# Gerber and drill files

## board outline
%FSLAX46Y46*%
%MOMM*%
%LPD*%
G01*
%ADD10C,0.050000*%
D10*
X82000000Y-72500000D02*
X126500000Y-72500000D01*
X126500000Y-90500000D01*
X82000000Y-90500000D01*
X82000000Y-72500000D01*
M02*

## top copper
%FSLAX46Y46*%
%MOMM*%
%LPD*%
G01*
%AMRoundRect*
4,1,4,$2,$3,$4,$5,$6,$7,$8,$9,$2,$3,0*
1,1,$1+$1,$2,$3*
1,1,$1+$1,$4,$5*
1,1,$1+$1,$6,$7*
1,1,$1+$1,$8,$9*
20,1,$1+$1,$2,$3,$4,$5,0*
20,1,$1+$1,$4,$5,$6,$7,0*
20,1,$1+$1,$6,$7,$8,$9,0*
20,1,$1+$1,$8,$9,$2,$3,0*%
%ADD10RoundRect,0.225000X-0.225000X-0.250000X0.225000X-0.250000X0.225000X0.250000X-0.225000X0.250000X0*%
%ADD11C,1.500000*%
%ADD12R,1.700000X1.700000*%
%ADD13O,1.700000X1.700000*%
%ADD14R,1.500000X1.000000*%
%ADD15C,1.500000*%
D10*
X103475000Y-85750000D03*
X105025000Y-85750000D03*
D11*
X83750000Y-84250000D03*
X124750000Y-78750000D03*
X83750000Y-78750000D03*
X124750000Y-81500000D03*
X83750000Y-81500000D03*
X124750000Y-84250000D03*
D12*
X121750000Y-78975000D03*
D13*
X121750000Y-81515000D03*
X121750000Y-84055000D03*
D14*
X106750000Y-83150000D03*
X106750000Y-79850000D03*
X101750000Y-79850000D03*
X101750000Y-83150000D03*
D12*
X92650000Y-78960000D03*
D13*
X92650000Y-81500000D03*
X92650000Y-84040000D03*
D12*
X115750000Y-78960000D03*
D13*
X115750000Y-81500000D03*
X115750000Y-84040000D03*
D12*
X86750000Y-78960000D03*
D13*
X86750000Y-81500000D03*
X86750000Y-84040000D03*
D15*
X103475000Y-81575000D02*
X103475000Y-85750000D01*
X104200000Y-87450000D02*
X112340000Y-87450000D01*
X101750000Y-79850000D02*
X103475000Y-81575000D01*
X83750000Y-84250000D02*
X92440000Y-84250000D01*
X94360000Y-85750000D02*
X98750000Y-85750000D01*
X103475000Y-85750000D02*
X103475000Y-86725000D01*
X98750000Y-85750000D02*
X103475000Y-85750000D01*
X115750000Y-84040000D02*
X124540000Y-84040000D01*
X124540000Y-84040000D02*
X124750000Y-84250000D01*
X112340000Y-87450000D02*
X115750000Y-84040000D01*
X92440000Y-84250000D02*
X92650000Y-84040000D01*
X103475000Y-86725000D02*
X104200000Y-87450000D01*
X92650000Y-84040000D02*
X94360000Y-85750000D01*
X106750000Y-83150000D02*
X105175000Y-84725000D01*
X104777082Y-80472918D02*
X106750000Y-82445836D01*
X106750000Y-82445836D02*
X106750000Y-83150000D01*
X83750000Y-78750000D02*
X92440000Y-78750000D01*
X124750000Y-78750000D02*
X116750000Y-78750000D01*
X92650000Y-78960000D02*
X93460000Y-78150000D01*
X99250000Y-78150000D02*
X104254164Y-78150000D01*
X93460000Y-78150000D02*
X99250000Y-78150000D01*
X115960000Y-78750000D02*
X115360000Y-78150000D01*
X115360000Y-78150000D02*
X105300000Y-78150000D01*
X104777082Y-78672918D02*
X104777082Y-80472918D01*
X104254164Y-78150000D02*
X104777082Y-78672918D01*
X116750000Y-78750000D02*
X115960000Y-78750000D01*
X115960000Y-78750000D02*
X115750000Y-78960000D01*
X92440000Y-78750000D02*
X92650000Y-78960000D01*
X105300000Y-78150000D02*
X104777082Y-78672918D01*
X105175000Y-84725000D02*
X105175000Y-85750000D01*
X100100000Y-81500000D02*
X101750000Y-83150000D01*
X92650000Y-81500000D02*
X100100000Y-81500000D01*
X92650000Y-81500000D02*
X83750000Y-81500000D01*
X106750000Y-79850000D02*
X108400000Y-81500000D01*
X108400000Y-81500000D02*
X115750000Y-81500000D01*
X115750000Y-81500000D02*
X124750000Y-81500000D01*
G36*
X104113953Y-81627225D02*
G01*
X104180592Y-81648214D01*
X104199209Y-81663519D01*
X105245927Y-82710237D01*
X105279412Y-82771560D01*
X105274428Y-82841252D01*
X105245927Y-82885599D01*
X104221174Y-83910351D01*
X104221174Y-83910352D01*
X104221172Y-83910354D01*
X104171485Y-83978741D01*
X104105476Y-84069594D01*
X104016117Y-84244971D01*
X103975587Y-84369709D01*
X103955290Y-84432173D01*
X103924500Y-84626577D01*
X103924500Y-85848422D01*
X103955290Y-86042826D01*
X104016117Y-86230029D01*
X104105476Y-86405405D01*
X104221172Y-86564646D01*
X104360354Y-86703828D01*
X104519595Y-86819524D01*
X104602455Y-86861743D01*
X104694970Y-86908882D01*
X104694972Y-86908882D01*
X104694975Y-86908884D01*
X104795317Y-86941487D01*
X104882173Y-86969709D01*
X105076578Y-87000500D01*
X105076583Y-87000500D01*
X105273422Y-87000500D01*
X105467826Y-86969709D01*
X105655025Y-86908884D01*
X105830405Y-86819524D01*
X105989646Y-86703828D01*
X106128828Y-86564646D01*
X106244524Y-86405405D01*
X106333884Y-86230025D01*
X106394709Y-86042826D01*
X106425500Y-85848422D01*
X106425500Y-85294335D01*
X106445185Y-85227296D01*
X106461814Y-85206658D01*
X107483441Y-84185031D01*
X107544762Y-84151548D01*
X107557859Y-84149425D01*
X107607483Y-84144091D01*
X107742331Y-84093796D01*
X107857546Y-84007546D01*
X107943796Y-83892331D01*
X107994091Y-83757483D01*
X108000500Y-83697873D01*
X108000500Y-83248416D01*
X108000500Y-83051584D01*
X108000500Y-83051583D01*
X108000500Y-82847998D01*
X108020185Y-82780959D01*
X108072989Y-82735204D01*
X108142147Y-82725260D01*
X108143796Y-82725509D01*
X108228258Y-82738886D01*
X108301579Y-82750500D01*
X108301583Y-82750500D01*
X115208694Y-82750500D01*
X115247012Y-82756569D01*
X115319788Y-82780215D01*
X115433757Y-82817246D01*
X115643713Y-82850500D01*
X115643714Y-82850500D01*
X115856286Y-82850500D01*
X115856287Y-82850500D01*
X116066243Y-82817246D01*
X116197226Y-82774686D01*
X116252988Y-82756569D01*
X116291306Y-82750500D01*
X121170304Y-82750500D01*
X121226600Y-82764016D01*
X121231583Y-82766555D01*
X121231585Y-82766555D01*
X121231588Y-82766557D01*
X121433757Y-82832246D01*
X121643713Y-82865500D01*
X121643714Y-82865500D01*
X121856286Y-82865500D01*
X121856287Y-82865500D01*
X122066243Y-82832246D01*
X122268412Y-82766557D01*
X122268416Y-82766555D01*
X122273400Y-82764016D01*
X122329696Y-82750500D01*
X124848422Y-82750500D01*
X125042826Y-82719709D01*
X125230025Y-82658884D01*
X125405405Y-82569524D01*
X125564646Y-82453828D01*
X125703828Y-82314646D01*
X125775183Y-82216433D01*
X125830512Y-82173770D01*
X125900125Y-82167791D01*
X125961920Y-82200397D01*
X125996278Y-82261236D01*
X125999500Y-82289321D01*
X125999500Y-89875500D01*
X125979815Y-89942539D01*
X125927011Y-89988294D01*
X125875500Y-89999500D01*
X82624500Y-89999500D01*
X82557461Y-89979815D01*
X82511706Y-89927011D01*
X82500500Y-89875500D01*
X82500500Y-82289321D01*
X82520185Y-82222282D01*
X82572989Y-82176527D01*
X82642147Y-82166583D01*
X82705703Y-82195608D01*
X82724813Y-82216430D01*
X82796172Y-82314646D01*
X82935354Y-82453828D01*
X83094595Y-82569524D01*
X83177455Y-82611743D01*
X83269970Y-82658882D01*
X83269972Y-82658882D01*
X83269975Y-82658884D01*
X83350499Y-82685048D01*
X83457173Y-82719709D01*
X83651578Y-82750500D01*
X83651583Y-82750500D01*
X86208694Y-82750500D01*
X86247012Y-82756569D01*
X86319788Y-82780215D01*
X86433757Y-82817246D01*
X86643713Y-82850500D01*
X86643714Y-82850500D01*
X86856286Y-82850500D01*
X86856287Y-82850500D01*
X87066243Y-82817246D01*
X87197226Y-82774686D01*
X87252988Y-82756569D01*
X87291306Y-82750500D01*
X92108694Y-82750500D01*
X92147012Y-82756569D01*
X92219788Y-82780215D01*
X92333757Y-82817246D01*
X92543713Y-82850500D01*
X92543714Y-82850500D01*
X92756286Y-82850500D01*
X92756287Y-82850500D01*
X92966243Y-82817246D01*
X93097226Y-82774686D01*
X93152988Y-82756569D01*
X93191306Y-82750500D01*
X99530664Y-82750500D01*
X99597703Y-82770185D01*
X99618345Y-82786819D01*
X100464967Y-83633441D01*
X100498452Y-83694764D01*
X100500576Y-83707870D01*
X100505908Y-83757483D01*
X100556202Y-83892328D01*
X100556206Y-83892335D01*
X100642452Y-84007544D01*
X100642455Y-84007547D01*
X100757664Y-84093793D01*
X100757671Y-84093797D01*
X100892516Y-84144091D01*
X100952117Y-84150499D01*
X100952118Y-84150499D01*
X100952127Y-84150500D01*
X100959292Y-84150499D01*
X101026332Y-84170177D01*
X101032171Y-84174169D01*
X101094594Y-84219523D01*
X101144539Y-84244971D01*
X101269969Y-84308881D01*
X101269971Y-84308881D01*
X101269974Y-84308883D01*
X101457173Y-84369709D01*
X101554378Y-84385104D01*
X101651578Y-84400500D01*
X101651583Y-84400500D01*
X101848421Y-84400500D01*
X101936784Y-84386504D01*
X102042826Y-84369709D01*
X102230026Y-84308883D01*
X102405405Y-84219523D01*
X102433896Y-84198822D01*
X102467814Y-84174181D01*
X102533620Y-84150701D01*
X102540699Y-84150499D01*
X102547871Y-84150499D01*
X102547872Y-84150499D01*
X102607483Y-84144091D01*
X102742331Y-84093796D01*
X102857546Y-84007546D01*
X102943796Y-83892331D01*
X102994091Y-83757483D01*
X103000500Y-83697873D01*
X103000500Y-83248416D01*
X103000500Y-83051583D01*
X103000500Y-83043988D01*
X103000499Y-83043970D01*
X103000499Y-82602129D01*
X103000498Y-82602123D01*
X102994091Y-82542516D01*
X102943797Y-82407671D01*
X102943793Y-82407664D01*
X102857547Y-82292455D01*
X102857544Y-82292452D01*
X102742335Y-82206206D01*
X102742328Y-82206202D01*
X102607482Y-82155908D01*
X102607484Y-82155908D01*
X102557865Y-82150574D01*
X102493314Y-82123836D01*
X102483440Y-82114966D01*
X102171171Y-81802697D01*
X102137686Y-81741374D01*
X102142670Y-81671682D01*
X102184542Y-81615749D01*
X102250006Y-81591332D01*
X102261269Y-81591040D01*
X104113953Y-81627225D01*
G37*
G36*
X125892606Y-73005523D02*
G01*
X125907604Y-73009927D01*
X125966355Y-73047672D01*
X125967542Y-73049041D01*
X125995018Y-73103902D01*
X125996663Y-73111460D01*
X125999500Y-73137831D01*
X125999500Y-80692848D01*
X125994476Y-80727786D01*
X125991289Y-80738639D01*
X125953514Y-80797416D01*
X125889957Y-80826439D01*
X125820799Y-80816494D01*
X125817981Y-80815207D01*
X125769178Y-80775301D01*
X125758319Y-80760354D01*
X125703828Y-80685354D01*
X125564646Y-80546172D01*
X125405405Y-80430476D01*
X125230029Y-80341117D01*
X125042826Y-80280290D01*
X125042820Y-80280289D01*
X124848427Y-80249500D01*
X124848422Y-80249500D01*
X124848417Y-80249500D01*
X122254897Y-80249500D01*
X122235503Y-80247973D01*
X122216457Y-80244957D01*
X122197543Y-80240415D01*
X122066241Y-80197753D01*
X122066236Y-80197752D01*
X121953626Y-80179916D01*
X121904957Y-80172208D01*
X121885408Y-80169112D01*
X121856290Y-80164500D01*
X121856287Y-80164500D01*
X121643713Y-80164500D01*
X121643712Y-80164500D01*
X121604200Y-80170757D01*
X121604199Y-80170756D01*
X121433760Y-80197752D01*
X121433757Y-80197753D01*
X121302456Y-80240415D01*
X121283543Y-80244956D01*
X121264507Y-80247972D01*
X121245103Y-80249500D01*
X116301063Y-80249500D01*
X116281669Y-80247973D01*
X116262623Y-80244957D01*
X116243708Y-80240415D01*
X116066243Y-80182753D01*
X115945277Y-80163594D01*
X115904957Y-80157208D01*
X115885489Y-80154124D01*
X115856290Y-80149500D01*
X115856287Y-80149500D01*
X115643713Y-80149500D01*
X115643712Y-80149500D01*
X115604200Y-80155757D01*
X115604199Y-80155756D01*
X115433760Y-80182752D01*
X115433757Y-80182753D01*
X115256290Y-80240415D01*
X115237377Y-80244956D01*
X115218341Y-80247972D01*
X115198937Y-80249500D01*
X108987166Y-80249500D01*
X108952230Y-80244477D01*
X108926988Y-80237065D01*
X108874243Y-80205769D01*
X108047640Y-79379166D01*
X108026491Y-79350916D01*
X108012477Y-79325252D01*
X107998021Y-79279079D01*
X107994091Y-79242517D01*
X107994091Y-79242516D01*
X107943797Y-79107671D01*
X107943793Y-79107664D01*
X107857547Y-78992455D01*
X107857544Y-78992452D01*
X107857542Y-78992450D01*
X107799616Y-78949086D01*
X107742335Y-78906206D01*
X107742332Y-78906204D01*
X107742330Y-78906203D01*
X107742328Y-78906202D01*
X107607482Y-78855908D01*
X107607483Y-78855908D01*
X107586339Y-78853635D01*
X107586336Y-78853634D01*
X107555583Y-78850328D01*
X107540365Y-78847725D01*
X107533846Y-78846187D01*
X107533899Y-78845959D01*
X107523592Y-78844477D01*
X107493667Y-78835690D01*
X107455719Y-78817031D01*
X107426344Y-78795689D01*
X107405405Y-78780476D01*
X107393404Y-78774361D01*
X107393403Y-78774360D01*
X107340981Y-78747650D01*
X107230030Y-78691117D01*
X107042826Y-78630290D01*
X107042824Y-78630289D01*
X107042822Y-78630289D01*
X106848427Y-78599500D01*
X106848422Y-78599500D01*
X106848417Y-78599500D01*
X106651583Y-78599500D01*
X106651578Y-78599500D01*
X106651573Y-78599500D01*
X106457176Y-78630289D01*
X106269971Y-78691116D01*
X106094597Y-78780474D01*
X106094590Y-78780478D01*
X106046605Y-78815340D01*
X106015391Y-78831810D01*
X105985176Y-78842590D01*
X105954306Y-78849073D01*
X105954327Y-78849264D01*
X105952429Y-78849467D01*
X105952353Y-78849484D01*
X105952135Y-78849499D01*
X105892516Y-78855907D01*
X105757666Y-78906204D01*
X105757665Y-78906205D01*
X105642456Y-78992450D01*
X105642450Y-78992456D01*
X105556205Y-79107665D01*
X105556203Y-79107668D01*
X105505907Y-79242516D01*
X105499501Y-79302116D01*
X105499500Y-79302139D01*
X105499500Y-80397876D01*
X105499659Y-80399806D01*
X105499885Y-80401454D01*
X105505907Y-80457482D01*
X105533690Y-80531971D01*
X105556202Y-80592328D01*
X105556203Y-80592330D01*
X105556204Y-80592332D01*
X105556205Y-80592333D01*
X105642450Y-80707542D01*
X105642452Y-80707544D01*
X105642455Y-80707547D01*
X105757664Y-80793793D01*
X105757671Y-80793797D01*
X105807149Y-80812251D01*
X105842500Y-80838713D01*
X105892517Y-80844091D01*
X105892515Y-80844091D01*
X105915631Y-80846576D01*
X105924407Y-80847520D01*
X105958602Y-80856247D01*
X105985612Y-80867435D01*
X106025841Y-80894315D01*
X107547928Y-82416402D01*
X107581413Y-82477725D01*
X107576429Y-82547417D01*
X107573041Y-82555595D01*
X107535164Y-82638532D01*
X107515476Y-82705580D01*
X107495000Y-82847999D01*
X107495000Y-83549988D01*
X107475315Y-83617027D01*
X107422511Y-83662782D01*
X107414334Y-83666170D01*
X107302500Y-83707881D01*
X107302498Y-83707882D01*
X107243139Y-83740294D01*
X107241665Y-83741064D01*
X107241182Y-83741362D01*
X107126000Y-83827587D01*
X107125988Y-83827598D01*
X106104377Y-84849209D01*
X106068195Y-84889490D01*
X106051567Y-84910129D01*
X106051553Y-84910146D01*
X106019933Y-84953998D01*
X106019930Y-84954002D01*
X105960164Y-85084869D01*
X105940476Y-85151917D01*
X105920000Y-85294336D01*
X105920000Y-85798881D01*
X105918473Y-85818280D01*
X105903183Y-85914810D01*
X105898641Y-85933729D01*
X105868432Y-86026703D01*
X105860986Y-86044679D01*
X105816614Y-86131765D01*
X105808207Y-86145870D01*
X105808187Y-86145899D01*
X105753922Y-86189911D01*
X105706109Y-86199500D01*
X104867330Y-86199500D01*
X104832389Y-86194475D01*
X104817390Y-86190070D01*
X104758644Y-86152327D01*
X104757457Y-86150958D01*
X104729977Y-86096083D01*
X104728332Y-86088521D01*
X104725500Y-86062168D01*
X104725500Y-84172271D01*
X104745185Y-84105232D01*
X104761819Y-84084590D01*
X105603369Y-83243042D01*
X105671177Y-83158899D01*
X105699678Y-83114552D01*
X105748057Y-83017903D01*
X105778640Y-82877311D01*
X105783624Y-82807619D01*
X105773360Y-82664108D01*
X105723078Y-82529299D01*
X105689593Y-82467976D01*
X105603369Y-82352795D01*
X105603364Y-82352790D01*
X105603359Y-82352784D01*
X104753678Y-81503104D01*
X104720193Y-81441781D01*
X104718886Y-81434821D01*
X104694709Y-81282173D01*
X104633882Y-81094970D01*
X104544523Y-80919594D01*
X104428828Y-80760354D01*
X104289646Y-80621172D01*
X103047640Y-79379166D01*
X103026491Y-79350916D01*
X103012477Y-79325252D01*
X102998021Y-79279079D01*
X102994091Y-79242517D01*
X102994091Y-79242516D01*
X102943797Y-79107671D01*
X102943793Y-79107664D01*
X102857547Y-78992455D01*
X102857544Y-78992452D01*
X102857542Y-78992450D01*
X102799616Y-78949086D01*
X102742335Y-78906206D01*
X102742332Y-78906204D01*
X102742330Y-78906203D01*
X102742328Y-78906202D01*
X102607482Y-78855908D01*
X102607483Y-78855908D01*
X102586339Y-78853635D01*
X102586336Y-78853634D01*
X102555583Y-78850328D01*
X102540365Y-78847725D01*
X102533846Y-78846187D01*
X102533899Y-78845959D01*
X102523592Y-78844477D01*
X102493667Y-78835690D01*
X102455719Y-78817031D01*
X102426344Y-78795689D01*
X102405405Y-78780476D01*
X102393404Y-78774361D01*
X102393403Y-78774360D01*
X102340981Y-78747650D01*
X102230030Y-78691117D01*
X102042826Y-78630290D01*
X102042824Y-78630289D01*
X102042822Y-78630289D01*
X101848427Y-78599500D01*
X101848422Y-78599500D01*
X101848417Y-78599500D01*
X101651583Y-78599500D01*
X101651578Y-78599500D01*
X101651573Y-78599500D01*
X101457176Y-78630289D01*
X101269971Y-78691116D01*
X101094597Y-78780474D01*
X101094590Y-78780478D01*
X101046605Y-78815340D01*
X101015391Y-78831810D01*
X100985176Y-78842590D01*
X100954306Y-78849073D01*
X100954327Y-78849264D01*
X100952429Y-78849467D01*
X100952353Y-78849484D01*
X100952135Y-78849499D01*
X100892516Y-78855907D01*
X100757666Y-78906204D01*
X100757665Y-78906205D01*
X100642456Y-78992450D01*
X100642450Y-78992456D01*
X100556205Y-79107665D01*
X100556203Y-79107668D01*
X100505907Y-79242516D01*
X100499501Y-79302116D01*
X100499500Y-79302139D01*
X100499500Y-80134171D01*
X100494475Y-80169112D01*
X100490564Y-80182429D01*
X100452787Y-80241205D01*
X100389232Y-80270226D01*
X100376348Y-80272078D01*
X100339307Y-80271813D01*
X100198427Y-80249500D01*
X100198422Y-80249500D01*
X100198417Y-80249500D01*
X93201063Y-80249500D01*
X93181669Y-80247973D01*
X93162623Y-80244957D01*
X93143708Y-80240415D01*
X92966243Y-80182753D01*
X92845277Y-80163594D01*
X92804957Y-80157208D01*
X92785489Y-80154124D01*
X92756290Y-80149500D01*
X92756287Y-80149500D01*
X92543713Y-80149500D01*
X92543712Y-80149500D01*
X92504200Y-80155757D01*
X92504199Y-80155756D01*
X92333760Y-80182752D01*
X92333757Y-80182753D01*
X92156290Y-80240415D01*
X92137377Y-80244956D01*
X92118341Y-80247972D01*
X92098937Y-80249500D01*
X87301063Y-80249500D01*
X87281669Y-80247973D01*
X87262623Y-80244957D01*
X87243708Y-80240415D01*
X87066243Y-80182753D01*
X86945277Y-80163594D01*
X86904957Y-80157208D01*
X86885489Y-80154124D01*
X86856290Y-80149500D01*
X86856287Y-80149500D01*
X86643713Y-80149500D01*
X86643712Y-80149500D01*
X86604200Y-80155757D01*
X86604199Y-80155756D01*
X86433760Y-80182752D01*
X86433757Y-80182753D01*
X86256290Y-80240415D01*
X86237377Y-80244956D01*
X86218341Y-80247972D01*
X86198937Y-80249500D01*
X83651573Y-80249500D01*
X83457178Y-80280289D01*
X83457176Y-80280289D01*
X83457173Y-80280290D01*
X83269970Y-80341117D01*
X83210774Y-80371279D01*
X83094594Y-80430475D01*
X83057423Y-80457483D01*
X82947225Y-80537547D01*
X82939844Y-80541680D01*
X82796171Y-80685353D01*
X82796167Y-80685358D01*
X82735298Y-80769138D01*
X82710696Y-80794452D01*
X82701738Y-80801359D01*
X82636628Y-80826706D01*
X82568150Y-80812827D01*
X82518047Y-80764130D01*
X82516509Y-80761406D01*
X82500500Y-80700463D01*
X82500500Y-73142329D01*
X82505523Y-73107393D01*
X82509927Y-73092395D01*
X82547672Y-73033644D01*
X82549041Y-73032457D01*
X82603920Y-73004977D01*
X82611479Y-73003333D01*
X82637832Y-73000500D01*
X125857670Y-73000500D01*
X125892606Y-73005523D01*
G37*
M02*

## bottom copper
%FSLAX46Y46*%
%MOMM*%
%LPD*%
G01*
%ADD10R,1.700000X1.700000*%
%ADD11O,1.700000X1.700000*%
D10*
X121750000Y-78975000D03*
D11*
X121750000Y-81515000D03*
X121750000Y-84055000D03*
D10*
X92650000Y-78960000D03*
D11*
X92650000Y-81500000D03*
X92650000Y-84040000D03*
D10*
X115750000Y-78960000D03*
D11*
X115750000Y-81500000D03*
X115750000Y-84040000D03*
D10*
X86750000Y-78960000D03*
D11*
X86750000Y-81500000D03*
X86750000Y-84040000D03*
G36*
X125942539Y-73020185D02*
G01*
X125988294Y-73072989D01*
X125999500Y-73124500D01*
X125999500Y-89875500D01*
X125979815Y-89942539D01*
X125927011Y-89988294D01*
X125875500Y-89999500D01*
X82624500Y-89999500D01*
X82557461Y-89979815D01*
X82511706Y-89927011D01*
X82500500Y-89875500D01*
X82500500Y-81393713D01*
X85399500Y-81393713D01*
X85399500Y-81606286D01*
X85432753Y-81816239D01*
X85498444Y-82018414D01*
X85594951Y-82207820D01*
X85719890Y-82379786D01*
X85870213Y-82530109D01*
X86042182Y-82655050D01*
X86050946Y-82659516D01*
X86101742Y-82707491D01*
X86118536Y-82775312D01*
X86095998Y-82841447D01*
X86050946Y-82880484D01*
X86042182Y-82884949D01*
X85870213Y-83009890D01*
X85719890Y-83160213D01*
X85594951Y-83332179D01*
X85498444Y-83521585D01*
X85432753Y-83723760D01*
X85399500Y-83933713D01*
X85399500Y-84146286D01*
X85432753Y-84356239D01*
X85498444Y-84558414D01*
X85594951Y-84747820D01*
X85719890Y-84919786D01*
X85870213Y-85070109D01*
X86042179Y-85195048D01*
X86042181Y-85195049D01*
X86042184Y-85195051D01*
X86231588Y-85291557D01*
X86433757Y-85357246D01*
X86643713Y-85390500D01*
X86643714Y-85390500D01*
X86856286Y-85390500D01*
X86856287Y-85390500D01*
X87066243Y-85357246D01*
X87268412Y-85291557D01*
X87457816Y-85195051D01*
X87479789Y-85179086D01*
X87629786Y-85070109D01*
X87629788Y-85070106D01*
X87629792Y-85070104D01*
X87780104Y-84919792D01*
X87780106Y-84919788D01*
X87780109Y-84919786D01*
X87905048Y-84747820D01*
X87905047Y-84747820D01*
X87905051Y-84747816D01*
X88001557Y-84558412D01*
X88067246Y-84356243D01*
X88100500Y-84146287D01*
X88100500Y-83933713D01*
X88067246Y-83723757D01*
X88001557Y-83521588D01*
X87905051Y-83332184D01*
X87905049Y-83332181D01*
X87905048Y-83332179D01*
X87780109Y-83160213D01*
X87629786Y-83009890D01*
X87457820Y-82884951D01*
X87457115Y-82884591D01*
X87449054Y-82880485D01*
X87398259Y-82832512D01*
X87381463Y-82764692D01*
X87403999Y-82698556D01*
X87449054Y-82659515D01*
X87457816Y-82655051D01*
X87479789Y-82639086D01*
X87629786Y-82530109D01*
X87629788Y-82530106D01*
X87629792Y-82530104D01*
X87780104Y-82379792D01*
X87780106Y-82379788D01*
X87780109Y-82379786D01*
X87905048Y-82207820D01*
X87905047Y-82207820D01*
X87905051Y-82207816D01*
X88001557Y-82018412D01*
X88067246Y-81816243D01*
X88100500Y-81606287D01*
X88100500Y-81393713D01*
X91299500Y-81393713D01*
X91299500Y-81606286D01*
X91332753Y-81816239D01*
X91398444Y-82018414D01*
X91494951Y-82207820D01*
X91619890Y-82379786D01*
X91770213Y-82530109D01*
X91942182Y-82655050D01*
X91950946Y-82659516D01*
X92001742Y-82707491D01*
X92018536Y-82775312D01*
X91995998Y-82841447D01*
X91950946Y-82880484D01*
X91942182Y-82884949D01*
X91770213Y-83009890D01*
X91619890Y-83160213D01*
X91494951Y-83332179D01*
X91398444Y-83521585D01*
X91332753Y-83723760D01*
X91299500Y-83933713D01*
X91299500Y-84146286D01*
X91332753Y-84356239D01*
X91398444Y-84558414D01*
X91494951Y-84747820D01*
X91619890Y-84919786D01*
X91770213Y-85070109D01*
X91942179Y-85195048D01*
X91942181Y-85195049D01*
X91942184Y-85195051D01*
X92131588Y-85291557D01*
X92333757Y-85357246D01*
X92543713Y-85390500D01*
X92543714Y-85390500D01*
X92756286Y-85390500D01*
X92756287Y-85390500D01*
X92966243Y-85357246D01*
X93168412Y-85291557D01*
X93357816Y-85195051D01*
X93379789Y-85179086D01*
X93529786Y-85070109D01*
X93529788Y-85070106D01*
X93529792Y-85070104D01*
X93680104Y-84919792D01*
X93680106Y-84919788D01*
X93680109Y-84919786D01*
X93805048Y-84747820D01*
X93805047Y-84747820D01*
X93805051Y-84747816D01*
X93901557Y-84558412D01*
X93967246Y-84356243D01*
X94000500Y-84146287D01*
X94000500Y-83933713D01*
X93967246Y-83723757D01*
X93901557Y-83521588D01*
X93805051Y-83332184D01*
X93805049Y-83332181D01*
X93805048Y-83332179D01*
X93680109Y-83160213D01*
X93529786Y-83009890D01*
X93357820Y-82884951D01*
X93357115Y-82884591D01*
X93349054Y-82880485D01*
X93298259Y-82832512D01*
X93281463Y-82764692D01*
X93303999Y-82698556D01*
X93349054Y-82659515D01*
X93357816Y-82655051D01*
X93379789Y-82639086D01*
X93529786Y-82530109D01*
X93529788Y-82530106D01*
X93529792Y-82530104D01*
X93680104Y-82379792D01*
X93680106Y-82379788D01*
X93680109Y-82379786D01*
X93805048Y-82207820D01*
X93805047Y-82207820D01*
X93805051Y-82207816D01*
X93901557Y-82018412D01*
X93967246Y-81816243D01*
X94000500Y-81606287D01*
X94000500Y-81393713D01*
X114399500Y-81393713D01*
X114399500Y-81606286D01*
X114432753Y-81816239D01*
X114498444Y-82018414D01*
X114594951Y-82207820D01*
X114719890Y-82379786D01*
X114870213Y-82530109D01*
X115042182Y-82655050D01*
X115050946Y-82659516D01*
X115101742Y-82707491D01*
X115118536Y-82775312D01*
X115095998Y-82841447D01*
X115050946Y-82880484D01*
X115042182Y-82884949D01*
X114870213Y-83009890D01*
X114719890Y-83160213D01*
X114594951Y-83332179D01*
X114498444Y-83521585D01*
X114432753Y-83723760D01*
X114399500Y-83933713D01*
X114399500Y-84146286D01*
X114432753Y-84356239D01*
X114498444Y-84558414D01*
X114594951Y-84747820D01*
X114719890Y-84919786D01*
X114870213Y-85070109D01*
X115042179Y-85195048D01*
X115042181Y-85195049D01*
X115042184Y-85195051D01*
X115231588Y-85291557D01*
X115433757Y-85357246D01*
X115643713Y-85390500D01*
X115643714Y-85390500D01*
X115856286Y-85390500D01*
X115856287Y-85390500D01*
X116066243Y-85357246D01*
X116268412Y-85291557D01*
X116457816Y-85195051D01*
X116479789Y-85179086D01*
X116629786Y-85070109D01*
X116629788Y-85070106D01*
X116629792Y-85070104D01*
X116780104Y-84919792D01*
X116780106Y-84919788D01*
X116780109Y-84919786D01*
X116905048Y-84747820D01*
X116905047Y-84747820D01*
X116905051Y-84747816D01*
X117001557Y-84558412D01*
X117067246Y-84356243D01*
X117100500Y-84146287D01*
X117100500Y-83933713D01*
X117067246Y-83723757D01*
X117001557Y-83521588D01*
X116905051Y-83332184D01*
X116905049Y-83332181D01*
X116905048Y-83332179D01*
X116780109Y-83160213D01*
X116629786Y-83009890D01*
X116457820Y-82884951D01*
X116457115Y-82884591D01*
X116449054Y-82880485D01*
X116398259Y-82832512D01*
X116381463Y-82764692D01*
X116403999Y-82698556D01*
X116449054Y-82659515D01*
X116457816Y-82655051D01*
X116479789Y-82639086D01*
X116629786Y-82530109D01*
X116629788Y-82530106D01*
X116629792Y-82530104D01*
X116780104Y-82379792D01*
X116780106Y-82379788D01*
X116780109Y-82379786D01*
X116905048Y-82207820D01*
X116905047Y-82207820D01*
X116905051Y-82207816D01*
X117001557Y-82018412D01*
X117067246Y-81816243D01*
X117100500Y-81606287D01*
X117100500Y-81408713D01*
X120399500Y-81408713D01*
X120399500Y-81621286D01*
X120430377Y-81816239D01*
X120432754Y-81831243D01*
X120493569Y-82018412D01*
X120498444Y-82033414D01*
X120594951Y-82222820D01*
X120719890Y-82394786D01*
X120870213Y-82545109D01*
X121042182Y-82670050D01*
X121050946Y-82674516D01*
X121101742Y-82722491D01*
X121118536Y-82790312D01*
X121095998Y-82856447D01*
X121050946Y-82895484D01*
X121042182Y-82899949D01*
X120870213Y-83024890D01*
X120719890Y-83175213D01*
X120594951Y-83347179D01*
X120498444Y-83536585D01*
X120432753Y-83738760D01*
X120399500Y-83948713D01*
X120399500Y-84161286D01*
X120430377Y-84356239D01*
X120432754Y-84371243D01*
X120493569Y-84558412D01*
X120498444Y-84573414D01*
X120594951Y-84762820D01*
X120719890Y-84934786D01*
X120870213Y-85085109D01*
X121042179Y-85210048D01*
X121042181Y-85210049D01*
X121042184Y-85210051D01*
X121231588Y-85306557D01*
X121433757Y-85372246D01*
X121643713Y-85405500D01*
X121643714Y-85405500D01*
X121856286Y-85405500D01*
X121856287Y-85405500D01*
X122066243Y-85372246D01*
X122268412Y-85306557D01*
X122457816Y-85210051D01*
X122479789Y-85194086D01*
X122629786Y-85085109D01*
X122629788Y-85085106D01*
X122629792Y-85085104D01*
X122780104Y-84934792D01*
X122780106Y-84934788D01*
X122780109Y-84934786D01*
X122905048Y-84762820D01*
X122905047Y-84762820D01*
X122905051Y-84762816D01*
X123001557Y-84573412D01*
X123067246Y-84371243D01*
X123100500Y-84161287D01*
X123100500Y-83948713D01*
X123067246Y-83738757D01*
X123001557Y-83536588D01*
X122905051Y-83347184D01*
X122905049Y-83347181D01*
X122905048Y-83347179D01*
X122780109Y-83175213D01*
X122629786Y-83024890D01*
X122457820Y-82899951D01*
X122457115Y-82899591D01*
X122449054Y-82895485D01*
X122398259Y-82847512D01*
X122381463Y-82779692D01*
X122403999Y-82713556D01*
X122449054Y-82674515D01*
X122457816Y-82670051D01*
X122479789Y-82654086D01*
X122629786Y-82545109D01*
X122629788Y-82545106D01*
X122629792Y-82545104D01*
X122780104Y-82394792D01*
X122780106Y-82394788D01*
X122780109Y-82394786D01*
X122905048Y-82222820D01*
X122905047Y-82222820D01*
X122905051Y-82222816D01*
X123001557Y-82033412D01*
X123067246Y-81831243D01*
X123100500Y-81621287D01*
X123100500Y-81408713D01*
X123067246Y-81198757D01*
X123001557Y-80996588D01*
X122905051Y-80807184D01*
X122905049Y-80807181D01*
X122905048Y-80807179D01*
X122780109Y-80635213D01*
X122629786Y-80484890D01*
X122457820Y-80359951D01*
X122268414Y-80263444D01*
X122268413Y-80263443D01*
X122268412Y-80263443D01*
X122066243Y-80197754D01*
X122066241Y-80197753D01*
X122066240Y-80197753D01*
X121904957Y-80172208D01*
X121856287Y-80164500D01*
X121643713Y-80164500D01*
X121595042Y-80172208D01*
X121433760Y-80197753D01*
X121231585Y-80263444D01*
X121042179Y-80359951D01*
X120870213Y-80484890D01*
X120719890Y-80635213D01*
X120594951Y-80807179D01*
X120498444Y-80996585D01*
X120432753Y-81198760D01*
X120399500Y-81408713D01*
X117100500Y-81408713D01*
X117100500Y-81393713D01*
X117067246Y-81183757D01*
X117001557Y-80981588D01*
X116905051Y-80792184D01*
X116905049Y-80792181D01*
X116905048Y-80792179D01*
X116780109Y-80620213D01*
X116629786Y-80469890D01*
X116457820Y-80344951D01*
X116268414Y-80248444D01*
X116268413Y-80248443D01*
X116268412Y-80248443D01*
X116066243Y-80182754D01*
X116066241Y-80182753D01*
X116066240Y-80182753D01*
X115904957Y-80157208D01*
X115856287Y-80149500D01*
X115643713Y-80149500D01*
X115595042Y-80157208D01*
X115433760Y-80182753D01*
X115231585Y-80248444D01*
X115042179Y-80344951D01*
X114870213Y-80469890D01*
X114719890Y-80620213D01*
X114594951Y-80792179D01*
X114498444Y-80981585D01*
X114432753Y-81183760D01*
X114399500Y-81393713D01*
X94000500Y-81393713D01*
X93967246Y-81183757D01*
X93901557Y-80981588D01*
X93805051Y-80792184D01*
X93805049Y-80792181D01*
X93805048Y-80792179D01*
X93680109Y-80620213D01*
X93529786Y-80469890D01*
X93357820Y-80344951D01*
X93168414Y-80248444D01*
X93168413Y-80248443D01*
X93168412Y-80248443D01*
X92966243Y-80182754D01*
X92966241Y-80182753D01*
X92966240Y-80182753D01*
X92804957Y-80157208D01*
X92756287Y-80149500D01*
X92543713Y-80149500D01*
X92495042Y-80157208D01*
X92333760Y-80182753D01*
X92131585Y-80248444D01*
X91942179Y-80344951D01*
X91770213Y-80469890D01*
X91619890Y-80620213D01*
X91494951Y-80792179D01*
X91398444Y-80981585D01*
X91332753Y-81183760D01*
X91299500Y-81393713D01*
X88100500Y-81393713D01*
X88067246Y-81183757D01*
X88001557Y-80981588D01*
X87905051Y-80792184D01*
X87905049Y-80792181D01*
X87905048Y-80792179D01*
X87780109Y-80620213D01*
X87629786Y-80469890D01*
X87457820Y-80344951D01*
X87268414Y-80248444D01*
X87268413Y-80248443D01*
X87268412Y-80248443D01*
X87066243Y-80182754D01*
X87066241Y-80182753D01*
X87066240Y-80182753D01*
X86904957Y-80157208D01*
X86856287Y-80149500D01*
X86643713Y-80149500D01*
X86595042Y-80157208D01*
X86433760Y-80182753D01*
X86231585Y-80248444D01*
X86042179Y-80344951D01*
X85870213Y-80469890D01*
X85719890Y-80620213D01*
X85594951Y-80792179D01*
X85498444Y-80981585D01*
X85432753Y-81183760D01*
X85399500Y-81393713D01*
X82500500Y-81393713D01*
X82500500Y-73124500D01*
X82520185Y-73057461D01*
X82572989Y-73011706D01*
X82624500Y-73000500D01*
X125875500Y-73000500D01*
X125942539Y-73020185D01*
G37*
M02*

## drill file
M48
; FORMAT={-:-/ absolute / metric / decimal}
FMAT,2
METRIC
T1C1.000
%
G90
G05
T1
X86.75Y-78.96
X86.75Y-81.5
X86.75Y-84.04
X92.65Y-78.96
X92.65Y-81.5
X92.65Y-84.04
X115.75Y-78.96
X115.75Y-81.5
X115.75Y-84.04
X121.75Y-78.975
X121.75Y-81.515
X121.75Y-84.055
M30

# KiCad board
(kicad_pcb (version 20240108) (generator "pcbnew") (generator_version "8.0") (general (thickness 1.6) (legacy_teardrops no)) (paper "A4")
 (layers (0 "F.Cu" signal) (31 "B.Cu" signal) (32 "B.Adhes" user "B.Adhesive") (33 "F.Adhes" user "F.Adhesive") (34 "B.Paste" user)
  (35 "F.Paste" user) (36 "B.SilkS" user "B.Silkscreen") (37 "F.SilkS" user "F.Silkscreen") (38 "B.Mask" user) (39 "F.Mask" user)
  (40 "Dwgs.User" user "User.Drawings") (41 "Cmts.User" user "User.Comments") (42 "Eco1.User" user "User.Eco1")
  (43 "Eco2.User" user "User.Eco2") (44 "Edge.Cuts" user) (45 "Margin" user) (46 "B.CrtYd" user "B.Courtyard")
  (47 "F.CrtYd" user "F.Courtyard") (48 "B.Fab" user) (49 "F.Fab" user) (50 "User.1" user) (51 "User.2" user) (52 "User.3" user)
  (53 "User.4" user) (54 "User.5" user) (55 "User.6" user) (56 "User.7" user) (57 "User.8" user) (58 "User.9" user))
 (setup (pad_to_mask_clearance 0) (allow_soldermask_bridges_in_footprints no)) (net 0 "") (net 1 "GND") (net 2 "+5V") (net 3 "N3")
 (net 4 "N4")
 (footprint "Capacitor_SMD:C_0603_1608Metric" (layer "F.Cu") (at 104.25 85.75)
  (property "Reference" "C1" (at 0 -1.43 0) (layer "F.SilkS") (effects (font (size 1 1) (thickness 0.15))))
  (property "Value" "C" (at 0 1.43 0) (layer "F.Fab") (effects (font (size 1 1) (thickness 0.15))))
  (pad "1" smd roundrect (at -0.775 0) (size 0.9 0.95) (layers "F.Cu" "F.Paste" "F.Mask") (roundrect_rratio 0.25) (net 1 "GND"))
  (pad "2" smd roundrect (at 0.775 0) (size 0.9 0.95) (layers "F.Cu" "F.Paste" "F.Mask") (roundrect_rratio 0.25) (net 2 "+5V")))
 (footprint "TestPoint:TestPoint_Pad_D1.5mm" (layer "F.Cu") (at 83.75 84.25 90)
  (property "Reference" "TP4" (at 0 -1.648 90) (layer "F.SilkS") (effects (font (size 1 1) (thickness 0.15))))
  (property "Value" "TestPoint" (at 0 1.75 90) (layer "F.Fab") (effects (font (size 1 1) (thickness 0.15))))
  (pad "1" smd circle (at 0 0 90) (size 1.5 1.5) (layers "F.Cu" "F.Mask") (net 1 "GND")))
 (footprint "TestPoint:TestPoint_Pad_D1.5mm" (layer "F.Cu") (at 124.75 78.75 90)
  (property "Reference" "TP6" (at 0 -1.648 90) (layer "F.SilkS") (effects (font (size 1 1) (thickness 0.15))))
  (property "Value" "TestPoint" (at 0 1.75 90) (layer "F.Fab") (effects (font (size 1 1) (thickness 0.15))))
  (pad "1" smd circle (at 0 0 90) (size 1.5 1.5) (layers "F.Cu" "F.Mask") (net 2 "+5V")))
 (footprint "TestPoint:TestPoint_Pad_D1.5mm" (layer "F.Cu") (at 83.75 78.75 90)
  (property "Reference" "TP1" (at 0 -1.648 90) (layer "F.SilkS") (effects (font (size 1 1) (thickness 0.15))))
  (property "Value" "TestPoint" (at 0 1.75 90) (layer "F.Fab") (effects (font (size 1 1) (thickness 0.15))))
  (pad "1" smd circle (at 0 0 90) (size 1.5 1.5) (layers "F.Cu" "F.Mask") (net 2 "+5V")))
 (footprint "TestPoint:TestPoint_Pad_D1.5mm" (layer "F.Cu") (at 124.75 81.5 90)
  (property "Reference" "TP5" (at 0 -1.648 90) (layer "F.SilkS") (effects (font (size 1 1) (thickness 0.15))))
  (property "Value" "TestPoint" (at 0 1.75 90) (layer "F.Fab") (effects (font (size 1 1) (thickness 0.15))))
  (pad "1" smd circle (at 0 0 90) (size 1.5 1.5) (layers "F.Cu" "F.Mask") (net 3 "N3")))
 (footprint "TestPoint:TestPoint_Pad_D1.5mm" (layer "F.Cu") (at 83.75 81.5 90)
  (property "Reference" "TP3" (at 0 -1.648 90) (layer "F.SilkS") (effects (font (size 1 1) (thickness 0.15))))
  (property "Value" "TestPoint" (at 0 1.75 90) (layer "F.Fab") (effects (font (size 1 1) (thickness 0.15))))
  (pad "1" smd circle (at 0 0 90) (size 1.5 1.5) (layers "F.Cu" "F.Mask") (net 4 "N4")))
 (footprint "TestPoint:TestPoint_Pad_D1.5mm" (layer "F.Cu") (at 124.75 84.25 90)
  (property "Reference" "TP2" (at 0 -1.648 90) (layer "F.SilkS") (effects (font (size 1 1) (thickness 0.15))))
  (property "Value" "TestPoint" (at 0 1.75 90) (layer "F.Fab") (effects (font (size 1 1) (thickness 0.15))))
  (pad "1" smd circle (at 0 0 90) (size 1.5 1.5) (layers "F.Cu" "F.Mask") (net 1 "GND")))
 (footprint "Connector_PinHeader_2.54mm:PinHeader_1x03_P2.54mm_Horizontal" (layer "F.Cu") (at 121.75 78.975)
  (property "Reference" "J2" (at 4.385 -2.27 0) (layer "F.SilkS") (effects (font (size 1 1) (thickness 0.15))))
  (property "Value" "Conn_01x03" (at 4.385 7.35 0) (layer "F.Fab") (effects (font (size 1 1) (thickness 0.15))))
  (pad "1" thru_hole rect (at 0 0) (size 1.7 1.7) (drill 1) (layers "*.Cu" "*.Mask") (remove_unused_layers no) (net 2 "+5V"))
  (pad "2" thru_hole oval (at 0 2.54) (size 1.7 1.7) (drill 1) (layers "*.Cu" "*.Mask") (remove_unused_layers no) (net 3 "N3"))
  (pad "3" thru_hole oval (at 0 5.08) (size 1.7 1.7) (drill 1) (layers "*.Cu" "*.Mask") (remove_unused_layers no) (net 1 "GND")))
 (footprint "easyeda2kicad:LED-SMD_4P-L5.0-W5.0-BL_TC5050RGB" (layer "F.Cu") (at 104.25 81.5 180)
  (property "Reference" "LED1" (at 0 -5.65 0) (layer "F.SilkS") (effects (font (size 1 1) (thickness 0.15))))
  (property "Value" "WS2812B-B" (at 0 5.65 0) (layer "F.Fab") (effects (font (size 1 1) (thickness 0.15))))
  (pad "1" smd rect (at -2.5 -1.65 180) (size 1.5 1) (layers "F.Cu" "F.Paste" "F.Mask") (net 2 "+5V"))
  (pad "2" smd rect (at -2.5 1.65 180) (size 1.5 1) (layers "F.Cu" "F.Paste" "F.Mask") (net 3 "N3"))
  (pad "3" smd rect (at 2.5 1.65 180) (size 1.5 1) (layers "F.Cu" "F.Paste" "F.Mask") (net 1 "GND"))
  (pad "4" smd rect (at 2.5 -1.65 180) (size 1.5 1) (layers "F.Cu" "F.Paste" "F.Mask") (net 4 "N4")))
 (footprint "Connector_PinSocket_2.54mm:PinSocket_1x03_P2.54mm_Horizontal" (layer "B.Cu") (at 92.65 78.96 180)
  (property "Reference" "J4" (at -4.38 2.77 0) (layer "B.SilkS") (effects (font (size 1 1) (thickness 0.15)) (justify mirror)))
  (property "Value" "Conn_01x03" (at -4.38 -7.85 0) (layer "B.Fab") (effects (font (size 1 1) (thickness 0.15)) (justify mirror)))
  (pad "1" thru_hole rect (at 0 0 180) (size 1.7 1.7) (drill 1) (layers "*.Cu" "*.Mask") (remove_unused_layers no) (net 2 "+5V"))
  (pad "2" thru_hole oval (at 0 -2.54 180) (size 1.7 1.7) (drill 1) (layers "*.Cu" "*.Mask") (remove_unused_layers no) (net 4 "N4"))
  (pad "3" thru_hole oval (at 0 -5.08 180) (size 1.7 1.7) (drill 1) (layers "*.Cu" "*.Mask") (remove_unused_layers no) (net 1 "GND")))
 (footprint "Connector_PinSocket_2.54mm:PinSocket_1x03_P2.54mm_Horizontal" (layer "B.Cu") (at 115.75 78.96 180)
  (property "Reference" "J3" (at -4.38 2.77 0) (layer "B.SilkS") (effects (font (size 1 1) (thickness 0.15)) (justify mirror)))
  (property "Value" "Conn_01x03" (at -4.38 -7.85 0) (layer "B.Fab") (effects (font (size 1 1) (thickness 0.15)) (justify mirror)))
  (pad "1" thru_hole rect (at 0 0 180) (size 1.7 1.7) (drill 1) (layers "*.Cu" "*.Mask") (remove_unused_layers no) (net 2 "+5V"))
  (pad "2" thru_hole oval (at 0 -2.54 180) (size 1.7 1.7) (drill 1) (layers "*.Cu" "*.Mask") (remove_unused_layers no) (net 3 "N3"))
  (pad "3" thru_hole oval (at 0 -5.08 180) (size 1.7 1.7) (drill 1) (layers "*.Cu" "*.Mask") (remove_unused_layers no) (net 1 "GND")))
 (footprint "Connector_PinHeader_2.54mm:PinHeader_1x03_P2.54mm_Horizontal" (layer "B.Cu") (at 86.75 78.96 180)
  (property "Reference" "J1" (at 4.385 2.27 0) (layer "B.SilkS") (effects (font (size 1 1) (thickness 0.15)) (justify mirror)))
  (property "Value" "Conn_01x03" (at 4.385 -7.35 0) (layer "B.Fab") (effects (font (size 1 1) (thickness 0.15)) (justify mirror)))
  (pad "1" thru_hole rect (at 0 0 180) (size 1.7 1.7) (drill 1) (layers "*.Cu" "*.Mask") (remove_unused_layers no) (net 2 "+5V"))
  (pad "2" thru_hole oval (at 0 -2.54 180) (size 1.7 1.7) (drill 1) (layers "*.Cu" "*.Mask") (remove_unused_layers no) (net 4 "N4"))
  (pad "3" thru_hole oval (at 0 -5.08 180) (size 1.7 1.7) (drill 1) (layers "*.Cu" "*.Mask") (remove_unused_layers no) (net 1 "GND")))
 (gr_rect (start 82 72.5) (end 126.5 90.5) (stroke (width 0.05) (type default)) (fill none) (layer "Edge.Cuts"))
 (segment (start 103.475 81.575) (end 103.475 85.75) (width 1.5) (layer "F.Cu") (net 1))
 (segment (start 104.2 87.45) (end 112.34 87.45) (width 1.5) (layer "F.Cu") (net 1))
 (segment (start 101.75 79.85) (end 103.475 81.575) (width 1.5) (layer "F.Cu") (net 1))
 (segment (start 83.75 84.25) (end 92.44 84.25) (width 1.5) (layer "F.Cu") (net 1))
 (segment (start 94.36 85.75) (end 98.75 85.75) (width 1.5) (layer "F.Cu") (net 1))
 (segment (start 103.475 85.75) (end 103.475 86.725) (width 1.5) (layer "F.Cu") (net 1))
 (segment (start 98.75 85.75) (end 103.475 85.75) (width 1.5) (layer "F.Cu") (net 1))
 (segment (start 115.75 84.04) (end 124.54 84.04) (width 1.5) (layer "F.Cu") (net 1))
 (segment (start 124.54 84.04) (end 124.75 84.25) (width 1.5) (layer "F.Cu") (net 1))
 (segment (start 112.34 87.45) (end 115.75 84.04) (width 1.5) (layer "F.Cu") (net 1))
 (segment (start 92.44 84.25) (end 92.65 84.04) (width 1.5) (layer "F.Cu") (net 1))
 (segment (start 103.475 86.725) (end 104.2 87.45) (width 1.5) (layer "F.Cu") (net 1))
 (segment (start 92.65 84.04) (end 94.36 85.75) (width 1.5) (layer "F.Cu") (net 1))
 (segment (start 106.75 83.15) (end 105.175 84.725) (width 1.5) (layer "F.Cu") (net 2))
 (segment (start 104.777082 80.472918) (end 106.75 82.445836) (width 1.5) (layer "F.Cu") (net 2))
 (segment (start 106.75 82.445836) (end 106.75 83.15) (width 1.5) (layer "F.Cu") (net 2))
 (segment (start 83.75 78.75) (end 92.44 78.75) (width 1.5) (layer "F.Cu") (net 2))
 (segment (start 124.75 78.75) (end 116.75 78.75) (width 1.5) (layer "F.Cu") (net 2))
 (segment (start 92.65 78.96) (end 93.46 78.15) (width 1.5) (layer "F.Cu") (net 2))
 (segment (start 99.25 78.15) (end 104.254164 78.15) (width 1.5) (layer "F.Cu") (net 2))
 (segment (start 93.46 78.15) (end 99.25 78.15) (width 1.5) (layer "F.Cu") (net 2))
 (segment (start 115.96 78.75) (end 115.36 78.15) (width 1.5) (layer "F.Cu") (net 2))
 (segment (start 115.36 78.15) (end 105.3 78.15) (width 1.5) (layer "F.Cu") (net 2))
 (segment (start 104.777082 78.672918) (end 104.777082 80.472918) (width 1.5) (layer "F.Cu") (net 2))
 (segment (start 104.254164 78.15) (end 104.777082 78.672918) (width 1.5) (layer "F.Cu") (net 2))
 (segment (start 116.75 78.75) (end 115.96 78.75) (width 1.5) (layer "F.Cu") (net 2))
 (segment (start 115.96 78.75) (end 115.75 78.96) (width 1.5) (layer "F.Cu") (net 2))
 (segment (start 92.44 78.75) (end 92.65 78.96) (width 1.5) (layer "F.Cu") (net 2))
 (segment (start 105.3 78.15) (end 104.777082 78.672918) (width 1.5) (layer "F.Cu") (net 2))
 (segment (start 105.175 84.725) (end 105.175 85.75) (width 1.5) (layer "F.Cu") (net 2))
 (segment (start 100.1 81.5) (end 101.75 83.15) (width 1.5) (layer "F.Cu") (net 4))
 (segment (start 92.65 81.5) (end 100.1 81.5) (width 1.5) (layer "F.Cu") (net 4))
 (segment (start 92.65 81.5) (end 83.75 81.5) (width 1.5) (layer "F.Cu") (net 4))
 (segment (start 106.75 79.85) (end 108.4 81.5) (width 1.5) (layer "F.Cu") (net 3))
 (segment (start 108.4 81.5) (end 115.75 81.5) (width 1.5) (layer "F.Cu") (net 3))
 (segment (start 115.75 81.5) (end 124.75 81.5) (width 1.5) (layer "F.Cu") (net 3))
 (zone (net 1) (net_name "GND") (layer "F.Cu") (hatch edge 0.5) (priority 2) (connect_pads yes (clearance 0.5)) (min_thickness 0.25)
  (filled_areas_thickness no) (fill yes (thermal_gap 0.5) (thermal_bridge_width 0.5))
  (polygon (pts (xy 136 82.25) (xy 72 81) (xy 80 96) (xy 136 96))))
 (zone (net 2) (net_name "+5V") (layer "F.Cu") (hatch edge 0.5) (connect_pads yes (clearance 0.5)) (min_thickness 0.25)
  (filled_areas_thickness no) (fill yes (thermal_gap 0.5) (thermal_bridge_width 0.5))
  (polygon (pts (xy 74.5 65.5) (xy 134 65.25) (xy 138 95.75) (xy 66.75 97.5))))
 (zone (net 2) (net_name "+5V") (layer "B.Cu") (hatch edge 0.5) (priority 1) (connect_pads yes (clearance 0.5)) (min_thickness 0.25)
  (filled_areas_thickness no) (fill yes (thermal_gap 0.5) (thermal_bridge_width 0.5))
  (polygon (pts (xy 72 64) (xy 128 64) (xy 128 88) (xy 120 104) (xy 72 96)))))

